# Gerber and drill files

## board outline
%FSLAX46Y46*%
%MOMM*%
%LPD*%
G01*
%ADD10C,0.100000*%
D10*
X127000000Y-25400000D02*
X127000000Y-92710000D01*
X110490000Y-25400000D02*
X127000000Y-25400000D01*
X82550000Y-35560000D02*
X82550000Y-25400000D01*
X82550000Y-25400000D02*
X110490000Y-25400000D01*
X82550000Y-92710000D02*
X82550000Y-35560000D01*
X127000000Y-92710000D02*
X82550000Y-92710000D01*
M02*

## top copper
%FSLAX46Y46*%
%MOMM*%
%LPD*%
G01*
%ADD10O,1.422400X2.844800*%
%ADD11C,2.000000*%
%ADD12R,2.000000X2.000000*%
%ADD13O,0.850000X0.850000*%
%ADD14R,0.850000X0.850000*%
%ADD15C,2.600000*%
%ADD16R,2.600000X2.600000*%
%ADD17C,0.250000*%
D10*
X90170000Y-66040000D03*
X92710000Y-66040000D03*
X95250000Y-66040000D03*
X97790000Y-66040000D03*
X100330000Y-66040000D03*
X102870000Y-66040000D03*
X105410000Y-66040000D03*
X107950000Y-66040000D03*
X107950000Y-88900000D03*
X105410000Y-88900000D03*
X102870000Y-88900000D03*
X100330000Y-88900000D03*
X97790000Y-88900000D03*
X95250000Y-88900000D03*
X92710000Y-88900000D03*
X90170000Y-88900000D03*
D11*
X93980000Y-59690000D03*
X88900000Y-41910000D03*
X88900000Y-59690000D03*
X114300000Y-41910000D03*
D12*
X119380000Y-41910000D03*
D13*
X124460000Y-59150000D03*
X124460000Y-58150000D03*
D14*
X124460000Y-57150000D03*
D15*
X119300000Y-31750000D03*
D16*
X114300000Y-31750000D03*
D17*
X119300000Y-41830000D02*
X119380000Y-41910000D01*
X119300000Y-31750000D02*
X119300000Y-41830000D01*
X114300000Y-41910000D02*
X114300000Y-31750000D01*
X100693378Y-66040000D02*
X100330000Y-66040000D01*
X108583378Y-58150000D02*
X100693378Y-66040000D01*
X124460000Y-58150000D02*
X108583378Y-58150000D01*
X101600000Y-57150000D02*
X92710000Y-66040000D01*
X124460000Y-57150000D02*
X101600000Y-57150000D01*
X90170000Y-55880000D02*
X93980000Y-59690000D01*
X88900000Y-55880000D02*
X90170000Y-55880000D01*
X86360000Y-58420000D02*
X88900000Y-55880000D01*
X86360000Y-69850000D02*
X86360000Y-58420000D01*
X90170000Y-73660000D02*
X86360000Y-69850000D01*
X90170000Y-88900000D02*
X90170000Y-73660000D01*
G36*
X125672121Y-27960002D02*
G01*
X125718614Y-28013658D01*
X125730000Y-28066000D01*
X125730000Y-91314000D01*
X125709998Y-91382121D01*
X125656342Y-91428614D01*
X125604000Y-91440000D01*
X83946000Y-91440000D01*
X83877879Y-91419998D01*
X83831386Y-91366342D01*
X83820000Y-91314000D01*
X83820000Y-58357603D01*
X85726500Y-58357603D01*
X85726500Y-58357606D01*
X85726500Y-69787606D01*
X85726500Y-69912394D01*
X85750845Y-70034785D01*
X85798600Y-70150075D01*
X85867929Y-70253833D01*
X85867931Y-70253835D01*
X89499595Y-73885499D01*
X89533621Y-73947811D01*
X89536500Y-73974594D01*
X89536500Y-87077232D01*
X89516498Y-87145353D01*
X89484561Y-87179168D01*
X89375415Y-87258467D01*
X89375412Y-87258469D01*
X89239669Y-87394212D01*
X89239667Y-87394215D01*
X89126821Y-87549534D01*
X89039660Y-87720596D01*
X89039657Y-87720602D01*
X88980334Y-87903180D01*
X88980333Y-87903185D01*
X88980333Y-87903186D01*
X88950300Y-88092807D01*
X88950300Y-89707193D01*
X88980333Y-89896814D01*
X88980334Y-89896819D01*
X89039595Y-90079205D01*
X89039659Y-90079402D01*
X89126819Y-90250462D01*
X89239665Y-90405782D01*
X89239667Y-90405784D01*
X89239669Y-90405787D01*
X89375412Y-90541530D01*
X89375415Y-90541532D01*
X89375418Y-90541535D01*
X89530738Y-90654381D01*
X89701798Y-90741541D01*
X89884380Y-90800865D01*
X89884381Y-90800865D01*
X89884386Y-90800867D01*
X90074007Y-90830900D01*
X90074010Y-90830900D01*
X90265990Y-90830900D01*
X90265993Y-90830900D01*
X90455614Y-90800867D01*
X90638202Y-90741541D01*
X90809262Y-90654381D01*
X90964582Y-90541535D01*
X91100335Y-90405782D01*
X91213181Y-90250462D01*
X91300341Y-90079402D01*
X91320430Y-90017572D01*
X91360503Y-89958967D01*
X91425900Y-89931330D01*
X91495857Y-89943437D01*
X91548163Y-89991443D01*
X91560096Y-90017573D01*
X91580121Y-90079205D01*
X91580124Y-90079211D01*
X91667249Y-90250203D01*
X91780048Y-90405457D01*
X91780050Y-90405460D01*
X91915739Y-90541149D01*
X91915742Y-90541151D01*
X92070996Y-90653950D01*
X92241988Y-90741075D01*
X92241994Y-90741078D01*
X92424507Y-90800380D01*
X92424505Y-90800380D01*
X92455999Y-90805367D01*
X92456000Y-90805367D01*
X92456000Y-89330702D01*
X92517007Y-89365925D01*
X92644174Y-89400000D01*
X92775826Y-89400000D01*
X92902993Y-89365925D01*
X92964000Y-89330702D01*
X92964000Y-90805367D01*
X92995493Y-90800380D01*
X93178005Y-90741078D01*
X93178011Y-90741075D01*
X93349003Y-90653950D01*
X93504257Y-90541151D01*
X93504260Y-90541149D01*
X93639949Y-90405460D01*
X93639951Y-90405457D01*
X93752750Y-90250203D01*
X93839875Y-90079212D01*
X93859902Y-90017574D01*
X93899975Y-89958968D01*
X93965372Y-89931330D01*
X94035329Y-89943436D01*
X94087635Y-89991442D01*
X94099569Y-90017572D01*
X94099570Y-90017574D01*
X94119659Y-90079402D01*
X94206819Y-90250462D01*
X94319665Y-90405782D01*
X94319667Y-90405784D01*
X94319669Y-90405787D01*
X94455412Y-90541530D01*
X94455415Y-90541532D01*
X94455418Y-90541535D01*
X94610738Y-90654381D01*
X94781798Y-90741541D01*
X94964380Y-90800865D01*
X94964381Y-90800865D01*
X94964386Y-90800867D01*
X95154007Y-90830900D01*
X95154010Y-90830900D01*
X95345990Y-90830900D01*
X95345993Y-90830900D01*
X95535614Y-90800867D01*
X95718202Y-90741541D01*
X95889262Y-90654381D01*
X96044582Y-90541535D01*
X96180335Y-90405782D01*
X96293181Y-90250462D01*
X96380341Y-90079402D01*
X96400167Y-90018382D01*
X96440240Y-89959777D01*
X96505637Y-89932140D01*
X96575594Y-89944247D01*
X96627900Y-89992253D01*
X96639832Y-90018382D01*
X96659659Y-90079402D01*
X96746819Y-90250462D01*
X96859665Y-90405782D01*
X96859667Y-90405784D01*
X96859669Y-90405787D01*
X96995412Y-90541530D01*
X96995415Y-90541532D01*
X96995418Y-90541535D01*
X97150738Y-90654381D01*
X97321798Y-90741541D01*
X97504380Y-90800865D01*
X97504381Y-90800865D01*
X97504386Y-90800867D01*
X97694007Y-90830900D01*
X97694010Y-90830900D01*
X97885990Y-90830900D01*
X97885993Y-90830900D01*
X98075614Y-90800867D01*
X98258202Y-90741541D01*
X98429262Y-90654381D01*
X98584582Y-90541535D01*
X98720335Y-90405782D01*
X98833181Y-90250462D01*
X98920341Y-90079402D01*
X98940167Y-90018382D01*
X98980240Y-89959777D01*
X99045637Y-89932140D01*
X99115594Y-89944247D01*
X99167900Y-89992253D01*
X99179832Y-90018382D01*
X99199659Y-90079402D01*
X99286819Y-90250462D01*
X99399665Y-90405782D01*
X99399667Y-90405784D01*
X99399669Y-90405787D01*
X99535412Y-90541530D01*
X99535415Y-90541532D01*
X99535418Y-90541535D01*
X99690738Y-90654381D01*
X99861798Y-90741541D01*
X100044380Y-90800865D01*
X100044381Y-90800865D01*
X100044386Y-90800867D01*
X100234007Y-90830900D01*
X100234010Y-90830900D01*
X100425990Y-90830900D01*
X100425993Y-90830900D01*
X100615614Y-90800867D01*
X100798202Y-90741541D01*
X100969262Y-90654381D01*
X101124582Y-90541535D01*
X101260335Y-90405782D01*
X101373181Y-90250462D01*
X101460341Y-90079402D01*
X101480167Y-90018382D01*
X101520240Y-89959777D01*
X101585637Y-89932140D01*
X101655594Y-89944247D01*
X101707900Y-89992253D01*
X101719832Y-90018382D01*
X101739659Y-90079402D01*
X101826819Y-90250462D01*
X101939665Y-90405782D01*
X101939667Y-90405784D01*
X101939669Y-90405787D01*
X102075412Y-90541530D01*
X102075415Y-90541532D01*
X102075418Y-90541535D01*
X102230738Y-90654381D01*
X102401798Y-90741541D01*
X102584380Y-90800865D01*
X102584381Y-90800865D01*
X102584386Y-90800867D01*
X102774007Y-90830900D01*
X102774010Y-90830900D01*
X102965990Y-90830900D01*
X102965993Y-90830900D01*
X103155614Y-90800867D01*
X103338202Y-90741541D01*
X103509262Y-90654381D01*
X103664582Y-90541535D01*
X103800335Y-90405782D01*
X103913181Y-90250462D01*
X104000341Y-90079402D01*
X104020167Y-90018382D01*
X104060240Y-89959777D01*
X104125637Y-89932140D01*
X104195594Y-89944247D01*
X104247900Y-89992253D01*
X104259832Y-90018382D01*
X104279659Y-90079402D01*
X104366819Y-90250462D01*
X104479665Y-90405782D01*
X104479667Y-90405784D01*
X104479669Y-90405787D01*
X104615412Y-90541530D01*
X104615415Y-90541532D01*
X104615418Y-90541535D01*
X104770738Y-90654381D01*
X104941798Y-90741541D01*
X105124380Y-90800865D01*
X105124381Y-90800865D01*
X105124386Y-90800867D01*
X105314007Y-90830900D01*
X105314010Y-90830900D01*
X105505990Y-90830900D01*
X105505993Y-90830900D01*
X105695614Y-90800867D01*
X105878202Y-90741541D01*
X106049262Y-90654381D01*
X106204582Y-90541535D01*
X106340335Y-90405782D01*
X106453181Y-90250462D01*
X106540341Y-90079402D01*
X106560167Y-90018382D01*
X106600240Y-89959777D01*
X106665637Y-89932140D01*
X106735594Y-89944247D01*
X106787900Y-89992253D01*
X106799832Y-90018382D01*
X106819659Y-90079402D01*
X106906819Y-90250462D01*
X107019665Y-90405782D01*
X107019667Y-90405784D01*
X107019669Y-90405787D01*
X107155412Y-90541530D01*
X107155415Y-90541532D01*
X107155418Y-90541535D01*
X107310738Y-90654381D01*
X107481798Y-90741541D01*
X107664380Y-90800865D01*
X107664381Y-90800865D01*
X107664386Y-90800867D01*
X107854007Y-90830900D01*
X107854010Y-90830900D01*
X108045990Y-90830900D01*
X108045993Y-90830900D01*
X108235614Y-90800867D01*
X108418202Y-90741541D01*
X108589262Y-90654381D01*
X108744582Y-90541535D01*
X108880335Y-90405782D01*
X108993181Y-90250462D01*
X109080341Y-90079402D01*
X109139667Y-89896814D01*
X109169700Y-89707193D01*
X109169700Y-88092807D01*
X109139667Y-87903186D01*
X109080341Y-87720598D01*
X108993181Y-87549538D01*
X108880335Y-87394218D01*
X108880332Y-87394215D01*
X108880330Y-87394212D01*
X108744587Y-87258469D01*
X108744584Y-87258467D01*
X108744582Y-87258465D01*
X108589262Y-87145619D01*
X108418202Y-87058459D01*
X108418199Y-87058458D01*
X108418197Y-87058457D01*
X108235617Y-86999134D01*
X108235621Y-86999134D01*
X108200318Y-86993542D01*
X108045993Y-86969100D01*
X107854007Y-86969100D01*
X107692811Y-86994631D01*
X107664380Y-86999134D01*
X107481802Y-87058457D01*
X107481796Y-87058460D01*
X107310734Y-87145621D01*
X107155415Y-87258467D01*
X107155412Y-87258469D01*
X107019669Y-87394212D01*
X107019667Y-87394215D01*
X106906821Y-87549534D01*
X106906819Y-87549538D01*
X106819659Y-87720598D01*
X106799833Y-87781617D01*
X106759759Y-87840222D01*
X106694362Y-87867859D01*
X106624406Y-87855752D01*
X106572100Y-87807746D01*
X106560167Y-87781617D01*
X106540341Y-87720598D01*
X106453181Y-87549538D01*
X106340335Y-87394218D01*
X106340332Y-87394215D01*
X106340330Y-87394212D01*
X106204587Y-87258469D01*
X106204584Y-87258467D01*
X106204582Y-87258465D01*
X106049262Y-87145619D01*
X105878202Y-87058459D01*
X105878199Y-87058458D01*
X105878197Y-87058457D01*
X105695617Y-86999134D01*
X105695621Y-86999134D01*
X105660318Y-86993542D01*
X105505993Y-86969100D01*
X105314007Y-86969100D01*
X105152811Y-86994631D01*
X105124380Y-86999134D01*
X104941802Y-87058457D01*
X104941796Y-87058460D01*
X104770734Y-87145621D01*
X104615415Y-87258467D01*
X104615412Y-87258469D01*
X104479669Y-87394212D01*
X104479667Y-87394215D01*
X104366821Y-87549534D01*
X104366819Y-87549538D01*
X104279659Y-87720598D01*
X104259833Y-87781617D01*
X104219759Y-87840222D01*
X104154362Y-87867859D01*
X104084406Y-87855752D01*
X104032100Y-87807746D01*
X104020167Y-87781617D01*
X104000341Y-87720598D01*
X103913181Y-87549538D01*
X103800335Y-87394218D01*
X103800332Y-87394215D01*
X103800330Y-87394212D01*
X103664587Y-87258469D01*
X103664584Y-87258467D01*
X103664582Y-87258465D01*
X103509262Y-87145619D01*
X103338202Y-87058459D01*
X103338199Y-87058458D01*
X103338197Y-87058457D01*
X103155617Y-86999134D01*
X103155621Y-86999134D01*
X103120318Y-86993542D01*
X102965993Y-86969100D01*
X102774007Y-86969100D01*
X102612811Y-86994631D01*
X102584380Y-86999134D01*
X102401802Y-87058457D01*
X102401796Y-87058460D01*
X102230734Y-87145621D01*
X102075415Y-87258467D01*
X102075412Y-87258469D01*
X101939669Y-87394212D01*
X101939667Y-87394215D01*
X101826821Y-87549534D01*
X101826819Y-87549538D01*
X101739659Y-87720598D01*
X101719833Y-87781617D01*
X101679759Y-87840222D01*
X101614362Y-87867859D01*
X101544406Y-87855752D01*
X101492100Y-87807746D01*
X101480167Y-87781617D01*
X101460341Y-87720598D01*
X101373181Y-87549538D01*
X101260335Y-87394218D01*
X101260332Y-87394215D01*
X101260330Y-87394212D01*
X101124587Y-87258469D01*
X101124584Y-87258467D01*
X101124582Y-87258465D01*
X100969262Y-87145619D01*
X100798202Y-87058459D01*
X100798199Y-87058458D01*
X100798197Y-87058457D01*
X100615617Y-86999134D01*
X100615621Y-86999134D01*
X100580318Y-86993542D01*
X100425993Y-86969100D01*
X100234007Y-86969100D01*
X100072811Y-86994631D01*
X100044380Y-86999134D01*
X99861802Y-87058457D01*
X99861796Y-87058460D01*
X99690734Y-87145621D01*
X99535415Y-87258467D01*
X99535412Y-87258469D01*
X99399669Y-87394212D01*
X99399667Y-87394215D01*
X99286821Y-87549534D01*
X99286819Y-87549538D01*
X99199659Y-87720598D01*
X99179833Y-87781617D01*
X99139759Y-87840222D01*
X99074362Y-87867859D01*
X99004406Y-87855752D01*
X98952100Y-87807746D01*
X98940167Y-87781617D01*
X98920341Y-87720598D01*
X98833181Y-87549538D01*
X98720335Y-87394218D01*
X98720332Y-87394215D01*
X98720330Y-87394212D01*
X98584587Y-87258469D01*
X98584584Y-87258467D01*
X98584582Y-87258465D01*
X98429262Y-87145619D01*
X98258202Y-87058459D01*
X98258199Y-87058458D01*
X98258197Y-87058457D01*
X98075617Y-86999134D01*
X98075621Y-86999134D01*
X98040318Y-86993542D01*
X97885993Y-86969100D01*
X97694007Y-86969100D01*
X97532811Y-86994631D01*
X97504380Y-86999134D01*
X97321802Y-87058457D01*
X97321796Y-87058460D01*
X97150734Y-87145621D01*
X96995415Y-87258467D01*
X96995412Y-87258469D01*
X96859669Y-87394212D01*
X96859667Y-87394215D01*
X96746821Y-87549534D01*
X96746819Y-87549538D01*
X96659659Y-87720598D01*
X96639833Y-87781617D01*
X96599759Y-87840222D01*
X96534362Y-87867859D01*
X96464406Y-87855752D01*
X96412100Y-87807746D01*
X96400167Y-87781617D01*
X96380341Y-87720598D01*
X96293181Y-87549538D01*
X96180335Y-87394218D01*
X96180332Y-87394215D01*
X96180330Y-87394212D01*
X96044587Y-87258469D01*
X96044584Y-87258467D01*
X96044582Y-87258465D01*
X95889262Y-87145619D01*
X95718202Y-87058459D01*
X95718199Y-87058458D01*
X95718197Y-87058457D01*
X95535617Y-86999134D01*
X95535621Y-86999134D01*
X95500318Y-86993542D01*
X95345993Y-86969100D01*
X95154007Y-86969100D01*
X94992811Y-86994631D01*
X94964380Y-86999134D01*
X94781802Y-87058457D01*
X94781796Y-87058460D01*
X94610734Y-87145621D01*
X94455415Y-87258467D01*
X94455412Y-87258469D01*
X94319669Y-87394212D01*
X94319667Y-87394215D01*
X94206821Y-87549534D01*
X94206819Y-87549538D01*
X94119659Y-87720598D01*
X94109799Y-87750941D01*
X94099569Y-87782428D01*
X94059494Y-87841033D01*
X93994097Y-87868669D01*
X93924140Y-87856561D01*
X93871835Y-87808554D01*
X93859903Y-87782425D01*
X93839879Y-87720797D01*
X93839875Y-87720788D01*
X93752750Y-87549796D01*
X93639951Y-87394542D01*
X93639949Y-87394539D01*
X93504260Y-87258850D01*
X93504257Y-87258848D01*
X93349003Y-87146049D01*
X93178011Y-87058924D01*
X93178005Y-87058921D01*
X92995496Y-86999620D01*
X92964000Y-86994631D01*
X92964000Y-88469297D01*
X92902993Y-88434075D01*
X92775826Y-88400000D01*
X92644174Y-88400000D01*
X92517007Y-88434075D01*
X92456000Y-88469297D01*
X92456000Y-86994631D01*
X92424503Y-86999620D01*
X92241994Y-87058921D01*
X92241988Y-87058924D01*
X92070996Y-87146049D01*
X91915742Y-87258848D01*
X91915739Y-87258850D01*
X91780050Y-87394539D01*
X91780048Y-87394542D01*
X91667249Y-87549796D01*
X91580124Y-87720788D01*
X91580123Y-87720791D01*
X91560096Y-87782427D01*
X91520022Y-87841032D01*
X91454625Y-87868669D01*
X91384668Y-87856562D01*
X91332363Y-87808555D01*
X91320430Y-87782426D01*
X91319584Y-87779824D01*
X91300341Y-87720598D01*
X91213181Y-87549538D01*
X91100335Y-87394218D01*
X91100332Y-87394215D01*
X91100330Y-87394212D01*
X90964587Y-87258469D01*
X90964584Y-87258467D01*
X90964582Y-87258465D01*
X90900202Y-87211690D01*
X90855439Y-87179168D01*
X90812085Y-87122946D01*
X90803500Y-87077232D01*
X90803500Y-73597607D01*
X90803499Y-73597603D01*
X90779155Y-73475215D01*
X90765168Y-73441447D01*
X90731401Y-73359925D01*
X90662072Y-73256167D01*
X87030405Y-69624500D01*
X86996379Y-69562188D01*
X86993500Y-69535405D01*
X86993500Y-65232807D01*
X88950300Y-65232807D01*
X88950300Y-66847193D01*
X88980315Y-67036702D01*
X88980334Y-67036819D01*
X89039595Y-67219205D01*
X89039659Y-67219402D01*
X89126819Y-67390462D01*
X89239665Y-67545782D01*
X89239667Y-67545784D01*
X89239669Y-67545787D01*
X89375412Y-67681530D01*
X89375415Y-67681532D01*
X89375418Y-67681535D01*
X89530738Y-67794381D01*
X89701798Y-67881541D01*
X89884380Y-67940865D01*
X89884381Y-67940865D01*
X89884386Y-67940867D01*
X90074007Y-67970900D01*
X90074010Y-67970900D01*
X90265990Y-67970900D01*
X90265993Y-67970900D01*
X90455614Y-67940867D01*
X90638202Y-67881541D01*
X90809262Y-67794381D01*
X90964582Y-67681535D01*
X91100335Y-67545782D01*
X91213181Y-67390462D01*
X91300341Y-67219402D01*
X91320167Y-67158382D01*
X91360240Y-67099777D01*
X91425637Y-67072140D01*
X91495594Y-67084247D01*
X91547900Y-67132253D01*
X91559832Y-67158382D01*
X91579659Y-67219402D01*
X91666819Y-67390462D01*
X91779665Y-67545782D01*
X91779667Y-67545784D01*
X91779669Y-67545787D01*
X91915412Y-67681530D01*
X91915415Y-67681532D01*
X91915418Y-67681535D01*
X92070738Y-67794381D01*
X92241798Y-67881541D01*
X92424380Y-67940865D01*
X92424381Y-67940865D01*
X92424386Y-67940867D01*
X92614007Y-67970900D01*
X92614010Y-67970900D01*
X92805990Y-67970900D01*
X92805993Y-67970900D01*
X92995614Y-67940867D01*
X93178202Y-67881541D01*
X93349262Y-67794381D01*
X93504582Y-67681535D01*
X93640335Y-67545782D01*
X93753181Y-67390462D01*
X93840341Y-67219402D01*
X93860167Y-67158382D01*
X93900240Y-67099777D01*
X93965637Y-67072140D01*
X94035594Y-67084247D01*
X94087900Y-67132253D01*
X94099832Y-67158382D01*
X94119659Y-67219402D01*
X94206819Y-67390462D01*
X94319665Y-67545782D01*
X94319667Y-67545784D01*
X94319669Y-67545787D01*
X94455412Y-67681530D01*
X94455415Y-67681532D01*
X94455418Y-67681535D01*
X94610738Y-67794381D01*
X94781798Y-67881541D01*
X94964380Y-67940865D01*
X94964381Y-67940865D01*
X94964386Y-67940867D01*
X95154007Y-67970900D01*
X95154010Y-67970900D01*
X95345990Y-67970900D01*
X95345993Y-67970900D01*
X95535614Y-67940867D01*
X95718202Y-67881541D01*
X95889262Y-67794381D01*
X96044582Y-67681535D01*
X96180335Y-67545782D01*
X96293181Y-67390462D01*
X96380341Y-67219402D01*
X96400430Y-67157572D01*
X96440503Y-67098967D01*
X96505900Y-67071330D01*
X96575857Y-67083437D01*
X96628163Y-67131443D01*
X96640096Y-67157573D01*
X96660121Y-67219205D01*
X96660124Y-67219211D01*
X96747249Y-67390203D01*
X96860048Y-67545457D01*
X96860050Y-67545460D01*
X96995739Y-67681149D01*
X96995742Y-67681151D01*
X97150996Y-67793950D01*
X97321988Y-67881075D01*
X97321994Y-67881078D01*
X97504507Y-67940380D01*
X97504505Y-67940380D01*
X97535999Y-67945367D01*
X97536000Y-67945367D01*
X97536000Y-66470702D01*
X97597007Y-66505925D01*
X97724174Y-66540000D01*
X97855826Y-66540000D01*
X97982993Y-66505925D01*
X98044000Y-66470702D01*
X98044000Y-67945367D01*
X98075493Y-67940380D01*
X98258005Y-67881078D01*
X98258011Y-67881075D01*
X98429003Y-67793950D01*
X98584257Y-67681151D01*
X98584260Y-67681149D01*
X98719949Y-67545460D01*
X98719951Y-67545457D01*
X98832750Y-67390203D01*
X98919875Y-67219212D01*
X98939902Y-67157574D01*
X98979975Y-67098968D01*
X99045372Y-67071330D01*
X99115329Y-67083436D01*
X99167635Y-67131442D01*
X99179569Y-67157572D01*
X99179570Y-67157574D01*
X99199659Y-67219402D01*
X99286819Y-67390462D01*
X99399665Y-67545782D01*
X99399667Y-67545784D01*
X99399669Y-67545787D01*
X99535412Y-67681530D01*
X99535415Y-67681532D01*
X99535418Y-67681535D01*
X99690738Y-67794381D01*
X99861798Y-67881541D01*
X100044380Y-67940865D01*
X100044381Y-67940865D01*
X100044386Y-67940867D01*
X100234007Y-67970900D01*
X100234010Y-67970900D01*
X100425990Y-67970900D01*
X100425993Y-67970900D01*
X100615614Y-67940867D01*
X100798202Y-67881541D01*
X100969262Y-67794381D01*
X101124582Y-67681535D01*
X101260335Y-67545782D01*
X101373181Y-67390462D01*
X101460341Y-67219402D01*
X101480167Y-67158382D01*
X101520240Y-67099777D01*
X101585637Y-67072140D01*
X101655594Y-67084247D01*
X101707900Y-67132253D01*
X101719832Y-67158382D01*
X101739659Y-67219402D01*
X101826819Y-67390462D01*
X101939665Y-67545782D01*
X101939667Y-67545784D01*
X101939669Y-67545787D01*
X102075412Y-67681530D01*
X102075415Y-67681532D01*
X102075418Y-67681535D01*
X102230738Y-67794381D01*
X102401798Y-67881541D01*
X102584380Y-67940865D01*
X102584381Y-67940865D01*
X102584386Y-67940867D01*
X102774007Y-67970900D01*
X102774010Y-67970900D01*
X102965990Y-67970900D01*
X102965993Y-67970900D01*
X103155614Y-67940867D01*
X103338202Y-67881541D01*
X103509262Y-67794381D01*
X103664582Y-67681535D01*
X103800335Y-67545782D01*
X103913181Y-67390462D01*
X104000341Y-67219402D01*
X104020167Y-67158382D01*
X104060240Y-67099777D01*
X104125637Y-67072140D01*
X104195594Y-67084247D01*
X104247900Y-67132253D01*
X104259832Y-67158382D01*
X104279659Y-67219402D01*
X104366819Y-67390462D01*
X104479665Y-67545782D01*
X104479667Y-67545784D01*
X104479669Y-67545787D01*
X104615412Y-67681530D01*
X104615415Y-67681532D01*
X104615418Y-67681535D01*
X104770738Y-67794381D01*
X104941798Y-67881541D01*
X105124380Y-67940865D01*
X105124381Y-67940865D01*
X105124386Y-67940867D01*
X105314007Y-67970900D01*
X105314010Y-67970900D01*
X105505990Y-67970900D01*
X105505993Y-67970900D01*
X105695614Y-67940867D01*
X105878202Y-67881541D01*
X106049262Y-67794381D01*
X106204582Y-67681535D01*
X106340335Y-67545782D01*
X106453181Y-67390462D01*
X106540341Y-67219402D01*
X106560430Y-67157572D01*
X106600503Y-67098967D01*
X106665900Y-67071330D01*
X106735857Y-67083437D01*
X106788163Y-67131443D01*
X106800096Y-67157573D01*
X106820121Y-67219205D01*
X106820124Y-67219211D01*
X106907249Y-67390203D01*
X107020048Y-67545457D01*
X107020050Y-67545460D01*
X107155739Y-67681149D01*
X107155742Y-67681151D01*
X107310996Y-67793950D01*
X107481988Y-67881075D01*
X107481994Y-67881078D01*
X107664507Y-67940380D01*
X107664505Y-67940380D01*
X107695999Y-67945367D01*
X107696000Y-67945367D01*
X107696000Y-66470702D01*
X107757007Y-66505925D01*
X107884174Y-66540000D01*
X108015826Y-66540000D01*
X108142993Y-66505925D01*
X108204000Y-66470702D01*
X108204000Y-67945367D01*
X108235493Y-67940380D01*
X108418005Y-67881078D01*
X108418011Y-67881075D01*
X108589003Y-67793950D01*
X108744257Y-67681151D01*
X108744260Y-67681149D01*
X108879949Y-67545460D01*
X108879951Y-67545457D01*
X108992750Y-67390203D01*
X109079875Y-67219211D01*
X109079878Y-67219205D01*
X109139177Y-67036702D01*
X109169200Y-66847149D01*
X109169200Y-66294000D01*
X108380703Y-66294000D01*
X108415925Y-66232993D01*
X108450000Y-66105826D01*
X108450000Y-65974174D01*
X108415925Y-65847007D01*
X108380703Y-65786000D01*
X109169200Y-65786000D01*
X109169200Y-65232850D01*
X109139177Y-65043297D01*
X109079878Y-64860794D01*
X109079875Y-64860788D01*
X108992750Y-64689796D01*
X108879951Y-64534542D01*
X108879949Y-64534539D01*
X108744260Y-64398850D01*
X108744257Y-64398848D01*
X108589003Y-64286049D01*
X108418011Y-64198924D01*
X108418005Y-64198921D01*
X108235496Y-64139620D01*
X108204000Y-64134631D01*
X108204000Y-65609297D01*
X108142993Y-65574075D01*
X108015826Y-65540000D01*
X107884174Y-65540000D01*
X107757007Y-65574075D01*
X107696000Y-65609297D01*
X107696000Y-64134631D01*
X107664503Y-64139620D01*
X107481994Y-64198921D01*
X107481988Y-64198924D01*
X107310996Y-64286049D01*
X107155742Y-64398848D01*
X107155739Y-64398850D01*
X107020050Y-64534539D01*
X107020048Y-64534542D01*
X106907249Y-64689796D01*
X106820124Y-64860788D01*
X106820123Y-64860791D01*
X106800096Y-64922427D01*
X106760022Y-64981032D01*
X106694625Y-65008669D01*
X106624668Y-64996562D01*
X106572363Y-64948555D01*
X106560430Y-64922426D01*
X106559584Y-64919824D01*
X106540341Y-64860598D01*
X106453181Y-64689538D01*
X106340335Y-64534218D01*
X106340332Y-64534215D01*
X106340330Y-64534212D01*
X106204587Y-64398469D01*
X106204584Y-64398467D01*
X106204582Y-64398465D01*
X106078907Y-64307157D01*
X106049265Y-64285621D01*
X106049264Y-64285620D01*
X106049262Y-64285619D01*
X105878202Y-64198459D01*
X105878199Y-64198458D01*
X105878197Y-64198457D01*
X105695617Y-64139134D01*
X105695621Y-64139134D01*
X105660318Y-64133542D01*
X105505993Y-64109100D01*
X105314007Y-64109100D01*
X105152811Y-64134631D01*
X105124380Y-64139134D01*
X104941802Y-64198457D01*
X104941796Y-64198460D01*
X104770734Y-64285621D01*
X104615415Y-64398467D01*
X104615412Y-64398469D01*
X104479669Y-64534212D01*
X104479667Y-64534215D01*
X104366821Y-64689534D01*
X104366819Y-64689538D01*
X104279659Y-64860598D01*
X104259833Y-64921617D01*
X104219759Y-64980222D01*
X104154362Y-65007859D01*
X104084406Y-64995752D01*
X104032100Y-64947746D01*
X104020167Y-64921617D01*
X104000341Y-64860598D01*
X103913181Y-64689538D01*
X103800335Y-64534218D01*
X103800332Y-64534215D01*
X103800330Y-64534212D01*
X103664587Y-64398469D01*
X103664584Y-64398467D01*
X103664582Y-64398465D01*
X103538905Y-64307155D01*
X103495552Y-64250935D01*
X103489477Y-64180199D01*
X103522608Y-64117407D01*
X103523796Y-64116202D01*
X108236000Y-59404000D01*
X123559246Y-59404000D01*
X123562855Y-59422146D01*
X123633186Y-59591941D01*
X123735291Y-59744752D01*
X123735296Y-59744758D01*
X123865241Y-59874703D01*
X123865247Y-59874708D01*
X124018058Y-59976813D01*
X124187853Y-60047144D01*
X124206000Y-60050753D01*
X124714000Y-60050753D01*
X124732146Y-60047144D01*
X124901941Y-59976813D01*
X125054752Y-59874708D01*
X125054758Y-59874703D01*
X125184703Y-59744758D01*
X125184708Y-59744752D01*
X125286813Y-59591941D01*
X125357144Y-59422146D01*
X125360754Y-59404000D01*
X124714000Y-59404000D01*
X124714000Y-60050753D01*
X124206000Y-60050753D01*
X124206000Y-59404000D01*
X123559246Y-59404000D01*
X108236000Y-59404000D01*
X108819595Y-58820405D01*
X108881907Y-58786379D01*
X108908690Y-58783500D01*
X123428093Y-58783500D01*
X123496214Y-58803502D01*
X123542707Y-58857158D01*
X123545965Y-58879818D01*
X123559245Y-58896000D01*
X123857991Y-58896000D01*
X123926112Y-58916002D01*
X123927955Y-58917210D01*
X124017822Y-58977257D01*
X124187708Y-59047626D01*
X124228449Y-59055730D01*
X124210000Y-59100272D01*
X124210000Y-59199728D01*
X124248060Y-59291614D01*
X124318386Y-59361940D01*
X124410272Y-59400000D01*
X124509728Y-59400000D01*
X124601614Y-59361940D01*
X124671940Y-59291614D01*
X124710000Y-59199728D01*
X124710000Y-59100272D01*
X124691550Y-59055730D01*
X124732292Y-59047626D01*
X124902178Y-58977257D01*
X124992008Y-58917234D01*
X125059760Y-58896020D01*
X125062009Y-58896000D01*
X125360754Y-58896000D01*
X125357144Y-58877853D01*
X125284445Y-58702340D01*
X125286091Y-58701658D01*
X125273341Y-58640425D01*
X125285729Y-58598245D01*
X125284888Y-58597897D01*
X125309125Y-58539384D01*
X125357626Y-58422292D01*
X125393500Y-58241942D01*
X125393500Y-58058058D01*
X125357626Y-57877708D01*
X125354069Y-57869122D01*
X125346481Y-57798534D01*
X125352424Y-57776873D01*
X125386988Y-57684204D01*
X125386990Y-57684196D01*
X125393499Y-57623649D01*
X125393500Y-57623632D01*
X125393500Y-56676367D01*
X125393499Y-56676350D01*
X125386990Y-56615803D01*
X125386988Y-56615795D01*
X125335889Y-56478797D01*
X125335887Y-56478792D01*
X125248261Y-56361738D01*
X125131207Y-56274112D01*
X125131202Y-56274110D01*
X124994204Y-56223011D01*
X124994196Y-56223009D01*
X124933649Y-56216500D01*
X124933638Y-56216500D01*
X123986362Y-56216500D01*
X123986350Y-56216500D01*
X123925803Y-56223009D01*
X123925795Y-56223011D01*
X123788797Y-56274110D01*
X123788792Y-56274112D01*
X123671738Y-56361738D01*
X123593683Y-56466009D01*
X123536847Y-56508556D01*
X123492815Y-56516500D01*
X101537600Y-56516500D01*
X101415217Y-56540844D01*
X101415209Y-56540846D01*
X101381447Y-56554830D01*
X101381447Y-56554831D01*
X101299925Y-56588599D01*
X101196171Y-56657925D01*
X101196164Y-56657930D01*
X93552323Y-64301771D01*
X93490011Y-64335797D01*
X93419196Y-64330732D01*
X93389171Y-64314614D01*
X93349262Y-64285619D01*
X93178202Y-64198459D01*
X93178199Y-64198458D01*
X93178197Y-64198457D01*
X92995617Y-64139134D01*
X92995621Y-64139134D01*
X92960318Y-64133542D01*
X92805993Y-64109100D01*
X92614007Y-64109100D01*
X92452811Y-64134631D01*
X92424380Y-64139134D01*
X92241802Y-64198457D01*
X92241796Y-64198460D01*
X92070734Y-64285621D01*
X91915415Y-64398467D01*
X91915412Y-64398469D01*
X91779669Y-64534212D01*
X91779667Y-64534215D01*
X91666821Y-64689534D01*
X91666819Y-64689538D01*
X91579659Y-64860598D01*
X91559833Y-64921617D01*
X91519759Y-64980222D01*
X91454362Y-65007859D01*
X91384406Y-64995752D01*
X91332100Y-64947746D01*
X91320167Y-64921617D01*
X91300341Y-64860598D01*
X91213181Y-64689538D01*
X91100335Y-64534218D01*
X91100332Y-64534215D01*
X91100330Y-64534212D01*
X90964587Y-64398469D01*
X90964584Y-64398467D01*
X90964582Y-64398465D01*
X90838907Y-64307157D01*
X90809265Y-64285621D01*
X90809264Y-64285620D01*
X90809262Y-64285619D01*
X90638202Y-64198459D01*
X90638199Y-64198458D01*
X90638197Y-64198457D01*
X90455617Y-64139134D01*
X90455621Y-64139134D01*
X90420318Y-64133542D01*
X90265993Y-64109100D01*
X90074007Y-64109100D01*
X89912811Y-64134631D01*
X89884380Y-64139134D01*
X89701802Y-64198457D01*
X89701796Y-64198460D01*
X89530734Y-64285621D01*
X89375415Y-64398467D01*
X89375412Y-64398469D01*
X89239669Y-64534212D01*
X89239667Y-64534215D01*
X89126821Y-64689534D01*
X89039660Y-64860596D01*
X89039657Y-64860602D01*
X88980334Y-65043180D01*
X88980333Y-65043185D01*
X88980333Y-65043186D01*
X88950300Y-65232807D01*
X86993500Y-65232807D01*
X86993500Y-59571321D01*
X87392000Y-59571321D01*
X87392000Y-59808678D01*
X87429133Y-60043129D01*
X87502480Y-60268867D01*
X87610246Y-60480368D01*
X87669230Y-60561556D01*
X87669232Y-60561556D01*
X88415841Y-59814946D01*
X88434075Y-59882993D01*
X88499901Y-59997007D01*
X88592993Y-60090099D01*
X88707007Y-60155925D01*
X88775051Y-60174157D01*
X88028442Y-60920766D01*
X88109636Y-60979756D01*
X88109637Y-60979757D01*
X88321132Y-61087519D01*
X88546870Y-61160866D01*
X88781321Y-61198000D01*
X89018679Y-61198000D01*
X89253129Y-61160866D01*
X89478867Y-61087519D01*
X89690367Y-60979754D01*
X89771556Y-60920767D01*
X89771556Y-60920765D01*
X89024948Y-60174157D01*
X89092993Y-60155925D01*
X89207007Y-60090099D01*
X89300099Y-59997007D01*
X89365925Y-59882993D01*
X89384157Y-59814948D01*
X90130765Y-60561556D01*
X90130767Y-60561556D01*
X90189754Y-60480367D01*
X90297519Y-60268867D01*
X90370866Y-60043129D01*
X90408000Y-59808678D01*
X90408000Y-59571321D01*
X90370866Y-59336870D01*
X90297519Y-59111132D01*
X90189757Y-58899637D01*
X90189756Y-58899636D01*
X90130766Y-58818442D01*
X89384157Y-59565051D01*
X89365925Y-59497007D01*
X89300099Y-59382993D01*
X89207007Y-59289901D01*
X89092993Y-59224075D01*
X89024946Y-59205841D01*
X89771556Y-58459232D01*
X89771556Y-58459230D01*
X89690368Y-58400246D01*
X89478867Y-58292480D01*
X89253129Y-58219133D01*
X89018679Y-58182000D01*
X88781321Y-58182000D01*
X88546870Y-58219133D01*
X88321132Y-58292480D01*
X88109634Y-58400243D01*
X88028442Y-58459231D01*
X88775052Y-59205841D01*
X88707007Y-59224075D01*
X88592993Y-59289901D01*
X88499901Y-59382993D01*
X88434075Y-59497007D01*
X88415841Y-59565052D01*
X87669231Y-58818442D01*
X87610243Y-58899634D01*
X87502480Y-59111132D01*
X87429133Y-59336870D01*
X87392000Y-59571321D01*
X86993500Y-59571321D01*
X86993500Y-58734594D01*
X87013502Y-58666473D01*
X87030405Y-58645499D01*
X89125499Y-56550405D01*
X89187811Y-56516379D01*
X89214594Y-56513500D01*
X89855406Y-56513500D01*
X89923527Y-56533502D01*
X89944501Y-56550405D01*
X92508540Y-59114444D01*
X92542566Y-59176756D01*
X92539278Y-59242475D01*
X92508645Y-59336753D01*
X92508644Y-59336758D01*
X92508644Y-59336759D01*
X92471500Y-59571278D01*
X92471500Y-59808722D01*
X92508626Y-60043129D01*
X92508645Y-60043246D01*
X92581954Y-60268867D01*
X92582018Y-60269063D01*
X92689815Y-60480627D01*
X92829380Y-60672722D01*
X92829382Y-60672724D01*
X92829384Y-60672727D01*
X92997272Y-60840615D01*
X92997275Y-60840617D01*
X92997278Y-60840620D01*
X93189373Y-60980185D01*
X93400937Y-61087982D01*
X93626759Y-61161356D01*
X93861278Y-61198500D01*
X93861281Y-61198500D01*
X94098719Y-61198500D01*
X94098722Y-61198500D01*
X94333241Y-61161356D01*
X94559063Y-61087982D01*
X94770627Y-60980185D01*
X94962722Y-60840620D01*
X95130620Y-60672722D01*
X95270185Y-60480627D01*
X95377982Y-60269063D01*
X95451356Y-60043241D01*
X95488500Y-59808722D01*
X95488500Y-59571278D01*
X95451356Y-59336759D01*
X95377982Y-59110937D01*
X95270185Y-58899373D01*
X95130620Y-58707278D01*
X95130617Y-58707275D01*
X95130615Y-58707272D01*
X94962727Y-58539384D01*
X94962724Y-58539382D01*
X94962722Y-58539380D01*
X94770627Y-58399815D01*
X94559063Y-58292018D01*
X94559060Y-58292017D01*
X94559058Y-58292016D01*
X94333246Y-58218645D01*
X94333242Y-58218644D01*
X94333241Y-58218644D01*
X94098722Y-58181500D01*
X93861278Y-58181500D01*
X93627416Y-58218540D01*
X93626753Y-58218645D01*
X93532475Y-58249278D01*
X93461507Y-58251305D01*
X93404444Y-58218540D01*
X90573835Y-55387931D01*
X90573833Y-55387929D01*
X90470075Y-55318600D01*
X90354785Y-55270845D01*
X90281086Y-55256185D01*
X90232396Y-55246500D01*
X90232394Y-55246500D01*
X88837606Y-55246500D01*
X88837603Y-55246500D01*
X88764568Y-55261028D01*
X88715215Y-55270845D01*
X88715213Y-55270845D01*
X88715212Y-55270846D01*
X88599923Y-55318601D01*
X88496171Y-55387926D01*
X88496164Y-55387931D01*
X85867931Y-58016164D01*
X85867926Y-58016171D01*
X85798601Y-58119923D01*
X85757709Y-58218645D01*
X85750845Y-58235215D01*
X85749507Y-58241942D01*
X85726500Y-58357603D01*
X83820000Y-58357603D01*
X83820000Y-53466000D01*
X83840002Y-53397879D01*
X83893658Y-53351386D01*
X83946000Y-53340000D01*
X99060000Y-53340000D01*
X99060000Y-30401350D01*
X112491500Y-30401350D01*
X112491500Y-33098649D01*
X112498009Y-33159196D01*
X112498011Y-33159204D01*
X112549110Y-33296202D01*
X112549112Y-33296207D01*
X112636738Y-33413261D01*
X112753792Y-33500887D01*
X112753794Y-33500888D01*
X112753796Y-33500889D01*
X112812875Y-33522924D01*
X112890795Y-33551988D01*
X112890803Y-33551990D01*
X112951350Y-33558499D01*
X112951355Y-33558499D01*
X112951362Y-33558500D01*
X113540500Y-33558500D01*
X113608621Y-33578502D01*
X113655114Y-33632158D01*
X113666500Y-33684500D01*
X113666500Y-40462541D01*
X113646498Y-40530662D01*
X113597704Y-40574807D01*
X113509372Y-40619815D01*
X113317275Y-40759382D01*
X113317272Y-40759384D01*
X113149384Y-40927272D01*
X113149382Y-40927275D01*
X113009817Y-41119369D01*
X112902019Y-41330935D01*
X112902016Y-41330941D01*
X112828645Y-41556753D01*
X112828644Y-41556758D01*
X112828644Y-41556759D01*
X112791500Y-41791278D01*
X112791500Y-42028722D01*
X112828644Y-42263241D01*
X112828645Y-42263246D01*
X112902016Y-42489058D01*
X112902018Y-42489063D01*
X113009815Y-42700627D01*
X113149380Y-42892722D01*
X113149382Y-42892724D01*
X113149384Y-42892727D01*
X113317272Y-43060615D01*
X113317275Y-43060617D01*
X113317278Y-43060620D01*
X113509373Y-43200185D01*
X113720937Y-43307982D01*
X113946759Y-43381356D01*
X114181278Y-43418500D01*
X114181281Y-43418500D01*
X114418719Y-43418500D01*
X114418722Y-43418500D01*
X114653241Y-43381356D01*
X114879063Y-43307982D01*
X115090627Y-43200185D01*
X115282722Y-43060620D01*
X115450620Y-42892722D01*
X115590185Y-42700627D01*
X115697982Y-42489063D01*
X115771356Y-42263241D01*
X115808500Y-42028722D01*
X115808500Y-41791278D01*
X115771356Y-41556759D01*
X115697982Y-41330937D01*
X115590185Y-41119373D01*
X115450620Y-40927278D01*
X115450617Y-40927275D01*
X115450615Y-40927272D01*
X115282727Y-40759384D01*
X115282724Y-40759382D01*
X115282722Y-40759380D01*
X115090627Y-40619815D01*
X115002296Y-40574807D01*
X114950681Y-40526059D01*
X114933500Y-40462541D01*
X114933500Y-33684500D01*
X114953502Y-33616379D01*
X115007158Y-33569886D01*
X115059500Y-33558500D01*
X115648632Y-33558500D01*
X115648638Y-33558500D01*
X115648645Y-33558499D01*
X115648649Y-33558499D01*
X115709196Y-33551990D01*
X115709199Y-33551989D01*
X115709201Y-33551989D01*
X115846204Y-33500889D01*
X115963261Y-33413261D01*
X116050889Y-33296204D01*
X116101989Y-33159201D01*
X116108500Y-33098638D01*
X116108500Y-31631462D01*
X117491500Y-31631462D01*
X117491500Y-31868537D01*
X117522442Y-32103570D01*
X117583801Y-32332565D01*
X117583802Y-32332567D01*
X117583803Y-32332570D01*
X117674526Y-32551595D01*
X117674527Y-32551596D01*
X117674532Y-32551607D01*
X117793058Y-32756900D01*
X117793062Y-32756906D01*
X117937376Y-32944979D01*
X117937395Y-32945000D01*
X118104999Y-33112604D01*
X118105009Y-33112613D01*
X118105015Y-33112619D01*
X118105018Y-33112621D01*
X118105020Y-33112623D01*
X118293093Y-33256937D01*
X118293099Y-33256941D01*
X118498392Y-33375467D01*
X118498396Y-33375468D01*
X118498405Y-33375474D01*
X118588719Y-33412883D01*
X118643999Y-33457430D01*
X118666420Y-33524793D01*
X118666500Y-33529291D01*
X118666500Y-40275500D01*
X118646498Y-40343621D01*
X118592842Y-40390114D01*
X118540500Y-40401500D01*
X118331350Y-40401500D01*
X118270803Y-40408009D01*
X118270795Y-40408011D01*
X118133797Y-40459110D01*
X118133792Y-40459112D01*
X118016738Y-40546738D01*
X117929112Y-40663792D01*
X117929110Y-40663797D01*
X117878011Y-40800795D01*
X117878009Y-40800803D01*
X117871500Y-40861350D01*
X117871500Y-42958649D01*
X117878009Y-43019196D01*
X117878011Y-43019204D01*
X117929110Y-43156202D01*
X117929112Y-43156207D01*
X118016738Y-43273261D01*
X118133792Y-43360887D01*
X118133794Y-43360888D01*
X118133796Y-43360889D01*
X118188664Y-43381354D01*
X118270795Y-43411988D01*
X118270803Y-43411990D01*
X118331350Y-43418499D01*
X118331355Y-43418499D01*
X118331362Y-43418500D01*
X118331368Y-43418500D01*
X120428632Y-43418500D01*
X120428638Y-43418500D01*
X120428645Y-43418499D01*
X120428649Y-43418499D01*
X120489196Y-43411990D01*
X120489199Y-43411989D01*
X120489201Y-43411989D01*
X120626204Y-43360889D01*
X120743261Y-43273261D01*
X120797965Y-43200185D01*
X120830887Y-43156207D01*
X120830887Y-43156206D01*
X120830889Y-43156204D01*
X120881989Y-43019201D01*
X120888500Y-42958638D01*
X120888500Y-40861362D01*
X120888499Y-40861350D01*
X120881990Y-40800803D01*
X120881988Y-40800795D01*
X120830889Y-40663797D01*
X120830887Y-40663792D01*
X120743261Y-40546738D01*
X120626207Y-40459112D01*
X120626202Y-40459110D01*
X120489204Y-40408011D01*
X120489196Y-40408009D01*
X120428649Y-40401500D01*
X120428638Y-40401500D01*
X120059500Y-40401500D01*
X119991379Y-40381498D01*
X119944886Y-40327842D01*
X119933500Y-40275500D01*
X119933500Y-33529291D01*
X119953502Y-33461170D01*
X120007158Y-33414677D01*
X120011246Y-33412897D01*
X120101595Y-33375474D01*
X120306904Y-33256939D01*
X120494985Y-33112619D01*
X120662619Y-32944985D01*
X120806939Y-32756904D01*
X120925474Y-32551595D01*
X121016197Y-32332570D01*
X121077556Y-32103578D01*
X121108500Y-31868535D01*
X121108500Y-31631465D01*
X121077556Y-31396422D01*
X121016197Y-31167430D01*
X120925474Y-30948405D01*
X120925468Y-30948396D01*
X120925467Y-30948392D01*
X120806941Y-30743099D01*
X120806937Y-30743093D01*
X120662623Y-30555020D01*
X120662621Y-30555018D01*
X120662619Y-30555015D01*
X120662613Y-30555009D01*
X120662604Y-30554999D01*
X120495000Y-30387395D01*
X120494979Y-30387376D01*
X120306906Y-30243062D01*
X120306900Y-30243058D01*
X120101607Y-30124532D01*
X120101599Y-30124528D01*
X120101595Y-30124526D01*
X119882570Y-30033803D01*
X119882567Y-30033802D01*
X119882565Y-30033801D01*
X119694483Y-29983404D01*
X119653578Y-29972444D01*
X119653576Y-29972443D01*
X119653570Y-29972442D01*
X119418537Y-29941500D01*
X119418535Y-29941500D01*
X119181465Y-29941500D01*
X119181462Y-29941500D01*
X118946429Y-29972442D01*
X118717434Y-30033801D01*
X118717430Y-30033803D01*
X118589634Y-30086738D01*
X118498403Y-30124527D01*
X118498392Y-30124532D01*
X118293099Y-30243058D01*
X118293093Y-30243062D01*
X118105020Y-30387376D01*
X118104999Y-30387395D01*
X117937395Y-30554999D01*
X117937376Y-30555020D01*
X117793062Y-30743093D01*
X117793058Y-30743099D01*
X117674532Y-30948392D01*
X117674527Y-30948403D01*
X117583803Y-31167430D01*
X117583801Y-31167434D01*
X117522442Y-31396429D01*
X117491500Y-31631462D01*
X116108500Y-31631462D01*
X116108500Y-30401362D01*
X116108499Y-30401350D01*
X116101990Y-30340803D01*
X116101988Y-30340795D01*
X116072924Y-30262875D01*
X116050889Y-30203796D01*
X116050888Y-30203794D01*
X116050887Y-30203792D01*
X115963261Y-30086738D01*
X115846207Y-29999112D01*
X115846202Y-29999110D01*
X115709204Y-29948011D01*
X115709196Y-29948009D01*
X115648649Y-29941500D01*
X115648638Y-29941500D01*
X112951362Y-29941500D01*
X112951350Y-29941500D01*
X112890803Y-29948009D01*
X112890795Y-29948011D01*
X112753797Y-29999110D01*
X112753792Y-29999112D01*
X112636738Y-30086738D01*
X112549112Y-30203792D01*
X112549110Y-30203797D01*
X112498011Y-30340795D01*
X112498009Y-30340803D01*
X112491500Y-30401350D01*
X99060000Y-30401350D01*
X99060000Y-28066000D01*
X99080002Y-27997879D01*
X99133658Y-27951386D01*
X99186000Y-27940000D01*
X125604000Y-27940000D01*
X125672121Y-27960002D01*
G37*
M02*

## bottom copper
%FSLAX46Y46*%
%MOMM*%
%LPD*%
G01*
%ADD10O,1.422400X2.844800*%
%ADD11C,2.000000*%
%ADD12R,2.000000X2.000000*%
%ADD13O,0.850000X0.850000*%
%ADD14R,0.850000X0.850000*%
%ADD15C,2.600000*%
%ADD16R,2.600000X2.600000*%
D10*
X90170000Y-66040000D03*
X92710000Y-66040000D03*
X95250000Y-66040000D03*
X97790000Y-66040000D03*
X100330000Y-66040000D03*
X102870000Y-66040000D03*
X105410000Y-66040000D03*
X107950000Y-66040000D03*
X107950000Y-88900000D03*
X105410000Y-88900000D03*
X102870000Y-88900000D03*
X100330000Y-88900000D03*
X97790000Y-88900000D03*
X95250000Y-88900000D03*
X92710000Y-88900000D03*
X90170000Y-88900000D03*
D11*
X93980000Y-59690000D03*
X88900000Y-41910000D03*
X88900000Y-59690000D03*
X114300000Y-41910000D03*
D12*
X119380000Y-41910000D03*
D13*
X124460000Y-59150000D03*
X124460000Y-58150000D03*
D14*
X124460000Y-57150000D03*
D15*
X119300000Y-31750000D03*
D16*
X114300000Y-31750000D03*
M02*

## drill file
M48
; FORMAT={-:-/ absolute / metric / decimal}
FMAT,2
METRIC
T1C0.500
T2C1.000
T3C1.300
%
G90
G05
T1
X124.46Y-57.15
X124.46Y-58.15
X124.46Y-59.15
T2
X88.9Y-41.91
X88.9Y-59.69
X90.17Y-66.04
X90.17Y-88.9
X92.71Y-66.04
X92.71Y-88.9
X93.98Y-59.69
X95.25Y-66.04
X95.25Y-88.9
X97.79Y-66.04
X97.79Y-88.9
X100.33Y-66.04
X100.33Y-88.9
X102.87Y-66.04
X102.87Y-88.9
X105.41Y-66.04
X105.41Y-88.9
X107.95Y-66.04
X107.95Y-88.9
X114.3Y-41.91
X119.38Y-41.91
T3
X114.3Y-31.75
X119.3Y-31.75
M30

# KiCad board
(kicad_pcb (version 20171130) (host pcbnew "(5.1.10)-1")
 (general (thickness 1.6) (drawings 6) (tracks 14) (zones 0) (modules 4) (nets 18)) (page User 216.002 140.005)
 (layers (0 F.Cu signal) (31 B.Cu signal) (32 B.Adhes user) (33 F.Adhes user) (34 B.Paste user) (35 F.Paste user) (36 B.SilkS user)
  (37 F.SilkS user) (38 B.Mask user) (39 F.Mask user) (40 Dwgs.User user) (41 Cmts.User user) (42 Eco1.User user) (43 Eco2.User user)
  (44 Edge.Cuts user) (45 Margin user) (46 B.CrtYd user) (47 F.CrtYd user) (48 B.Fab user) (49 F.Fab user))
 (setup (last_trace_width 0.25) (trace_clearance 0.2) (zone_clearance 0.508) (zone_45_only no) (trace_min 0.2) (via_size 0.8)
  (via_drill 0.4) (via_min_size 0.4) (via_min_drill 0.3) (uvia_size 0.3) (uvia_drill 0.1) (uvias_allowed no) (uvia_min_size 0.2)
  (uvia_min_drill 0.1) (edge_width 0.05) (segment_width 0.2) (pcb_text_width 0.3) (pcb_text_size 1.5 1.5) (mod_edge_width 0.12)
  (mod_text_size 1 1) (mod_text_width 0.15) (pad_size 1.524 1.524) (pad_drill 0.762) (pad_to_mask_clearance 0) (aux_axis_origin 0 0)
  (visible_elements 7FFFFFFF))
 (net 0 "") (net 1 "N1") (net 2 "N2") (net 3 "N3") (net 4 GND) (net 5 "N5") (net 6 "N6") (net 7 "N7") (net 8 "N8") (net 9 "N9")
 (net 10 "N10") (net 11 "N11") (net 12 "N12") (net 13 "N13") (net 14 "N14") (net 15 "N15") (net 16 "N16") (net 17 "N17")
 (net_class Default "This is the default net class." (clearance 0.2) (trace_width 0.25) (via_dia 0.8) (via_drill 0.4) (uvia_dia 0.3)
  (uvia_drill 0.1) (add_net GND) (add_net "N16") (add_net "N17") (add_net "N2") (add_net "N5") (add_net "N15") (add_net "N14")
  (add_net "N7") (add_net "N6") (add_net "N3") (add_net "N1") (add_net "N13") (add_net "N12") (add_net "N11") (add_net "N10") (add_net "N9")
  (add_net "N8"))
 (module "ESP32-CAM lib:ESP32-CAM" (layer F.Cu) (at 100.33 77.47 90)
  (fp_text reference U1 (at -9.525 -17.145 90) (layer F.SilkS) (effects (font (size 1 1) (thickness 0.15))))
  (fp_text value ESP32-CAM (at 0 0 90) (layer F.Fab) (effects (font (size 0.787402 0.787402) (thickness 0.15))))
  (pad P$16 thru_hole oval (at 11.43 -10.16 90) (size 2.8448 1.4224) (drill 1) (layers *.Cu *.Mask) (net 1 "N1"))
  (pad P$15 thru_hole oval (at 11.43 -7.62 90) (size 2.8448 1.4224) (drill 1) (layers *.Cu *.Mask) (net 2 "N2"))
  (pad P$14 thru_hole oval (at 11.43 -5.08 90) (size 2.8448 1.4224) (drill 1) (layers *.Cu *.Mask) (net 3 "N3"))
  (pad P$13 thru_hole oval (at 11.43 -2.54 90) (size 2.8448 1.4224) (drill 1) (layers *.Cu *.Mask) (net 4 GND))
  (pad P$12 thru_hole oval (at 11.43 0 90) (size 2.8448 1.4224) (drill 1) (layers *.Cu *.Mask) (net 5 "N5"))
  (pad P$11 thru_hole oval (at 11.43 2.54 90) (size 2.8448 1.4224) (drill 1) (layers *.Cu *.Mask) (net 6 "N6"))
  (pad P$10 thru_hole oval (at 11.43 5.08 90) (size 2.8448 1.4224) (drill 1) (layers *.Cu *.Mask) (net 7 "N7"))
  (pad P$9 thru_hole oval (at 11.43 7.62 90) (size 2.8448 1.4224) (drill 1) (layers *.Cu *.Mask) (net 4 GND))
  (pad P$8 thru_hole oval (at -11.43 7.62 90) (size 2.8448 1.4224) (drill 1) (layers *.Cu *.Mask) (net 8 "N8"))
  (pad P$7 thru_hole oval (at -11.43 5.08 90) (size 2.8448 1.4224) (drill 1) (layers *.Cu *.Mask) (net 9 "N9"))
  (pad P$6 thru_hole oval (at -11.43 2.54 90) (size 2.8448 1.4224) (drill 1) (layers *.Cu *.Mask) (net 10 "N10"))
  (pad P$5 thru_hole oval (at -11.43 0 90) (size 2.8448 1.4224) (drill 1) (layers *.Cu *.Mask) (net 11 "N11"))
  (pad P$4 thru_hole oval (at -11.43 -2.54 90) (size 2.8448 1.4224) (drill 1) (layers *.Cu *.Mask) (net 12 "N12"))
  (pad P$3 thru_hole oval (at -11.43 -5.08 90) (size 2.8448 1.4224) (drill 1) (layers *.Cu *.Mask) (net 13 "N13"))
  (pad P$2 thru_hole oval (at -11.43 -7.62 90) (size 2.8448 1.4224) (drill 1) (layers *.Cu *.Mask) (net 4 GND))
  (pad P$1 thru_hole oval (at -11.43 -10.16 90) (size 2.8448 1.4224) (drill 1) (layers *.Cu *.Mask) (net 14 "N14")))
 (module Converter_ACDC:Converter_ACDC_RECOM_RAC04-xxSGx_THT (layer F.Cu) (at 119.38 41.91 270)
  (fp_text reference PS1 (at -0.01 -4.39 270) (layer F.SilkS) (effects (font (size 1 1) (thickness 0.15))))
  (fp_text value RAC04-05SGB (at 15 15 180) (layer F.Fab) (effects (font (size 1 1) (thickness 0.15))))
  (pad 5 thru_hole circle (at 17.78 25.4) (size 2 2) (drill 1) (layers *.Cu *.Mask) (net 14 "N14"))
  (pad 3 thru_hole circle (at 0 30.48 90) (size 2 2) (drill 1) (layers *.Cu *.Mask) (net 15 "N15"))
  (pad 4 thru_hole circle (at 17.78 30.48) (size 2 2) (drill 1) (layers *.Cu *.Mask) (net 4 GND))
  (pad 2 thru_hole circle (at 0 5.08) (size 2 2) (drill 1) (layers *.Cu *.Mask) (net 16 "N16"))
  (pad 1 thru_hole rect (at 0 0) (size 2 2) (drill 1) (layers *.Cu *.Mask) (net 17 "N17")))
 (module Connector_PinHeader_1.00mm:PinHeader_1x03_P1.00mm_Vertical (layer F.Cu) (at 124.46 57.15)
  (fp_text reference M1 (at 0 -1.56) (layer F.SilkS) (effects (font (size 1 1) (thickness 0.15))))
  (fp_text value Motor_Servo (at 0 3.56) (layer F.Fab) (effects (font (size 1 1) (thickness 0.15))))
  (pad 3 thru_hole oval (at 0 2) (size 0.85 0.85) (drill 0.5) (layers *.Cu *.Mask) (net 4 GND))
  (pad 2 thru_hole oval (at 0 1) (size 0.85 0.85) (drill 0.5) (layers *.Cu *.Mask) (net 5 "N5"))
  (pad 1 thru_hole rect (at 0 0) (size 0.85 0.85) (drill 0.5) (layers *.Cu *.Mask) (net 2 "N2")))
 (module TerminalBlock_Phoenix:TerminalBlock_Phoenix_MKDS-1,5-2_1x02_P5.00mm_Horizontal (layer F.Cu) (at 114.3 31.75)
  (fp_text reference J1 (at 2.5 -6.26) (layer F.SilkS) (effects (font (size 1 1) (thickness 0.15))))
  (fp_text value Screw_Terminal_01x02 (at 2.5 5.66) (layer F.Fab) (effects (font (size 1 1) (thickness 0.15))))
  (pad 2 thru_hole circle (at 5 0) (size 2.6 2.6) (drill 1.3) (layers *.Cu *.Mask) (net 17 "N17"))
  (pad 1 thru_hole rect (at 0 0) (size 2.6 2.6) (drill 1.3) (layers *.Cu *.Mask) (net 16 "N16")))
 (gr_line (start 127 25.4) (end 127 92.71) (layer Edge.Cuts) (width 0.1))
 (gr_line (start 110.49 25.4) (end 127 25.4) (layer Edge.Cuts) (width 0.1))
 (gr_line (start 82.55 35.56) (end 82.55 25.4) (layer Edge.Cuts) (width 0.1))
 (gr_line (start 82.55 25.4) (end 110.49 25.4) (layer Edge.Cuts) (width 0.1))
 (gr_line (start 82.55 92.71) (end 82.55 35.56) (layer Edge.Cuts) (width 0.1))
 (gr_line (start 127 92.71) (end 82.55 92.71) (layer Edge.Cuts) (width 0.1))
 (segment (start 119.3 41.83) (end 119.38 41.91) (width 0.25) (layer F.Cu) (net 17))
 (segment (start 119.3 31.75) (end 119.3 41.83) (width 0.25) (layer F.Cu) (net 17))
 (segment (start 114.3 41.91) (end 114.3 31.75) (width 0.25) (layer F.Cu) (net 16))
 (segment (start 100.693378 66.04) (end 100.33 66.04) (width 0.25) (layer F.Cu) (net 5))
 (segment (start 108.583378 58.15) (end 100.693378 66.04) (width 0.25) (layer F.Cu) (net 5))
 (segment (start 124.46 58.15) (end 108.583378 58.15) (width 0.25) (layer F.Cu) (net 5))
 (segment (start 101.6 57.15) (end 92.71 66.04) (width 0.25) (layer F.Cu) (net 2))
 (segment (start 124.46 57.15) (end 101.6 57.15) (width 0.25) (layer F.Cu) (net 2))
 (segment (start 90.17 55.88) (end 93.98 59.69) (width 0.25) (layer F.Cu) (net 14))
 (segment (start 88.9 55.88) (end 90.17 55.88) (width 0.25) (layer F.Cu) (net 14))
 (segment (start 86.36 58.42) (end 88.9 55.88) (width 0.25) (layer F.Cu) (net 14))
 (segment (start 86.36 69.85) (end 86.36 58.42) (width 0.25) (layer F.Cu) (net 14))
 (segment (start 90.17 73.66) (end 86.36 69.85) (width 0.25) (layer F.Cu) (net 14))
 (segment (start 90.17 88.9) (end 90.17 73.66) (width 0.25) (layer F.Cu) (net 14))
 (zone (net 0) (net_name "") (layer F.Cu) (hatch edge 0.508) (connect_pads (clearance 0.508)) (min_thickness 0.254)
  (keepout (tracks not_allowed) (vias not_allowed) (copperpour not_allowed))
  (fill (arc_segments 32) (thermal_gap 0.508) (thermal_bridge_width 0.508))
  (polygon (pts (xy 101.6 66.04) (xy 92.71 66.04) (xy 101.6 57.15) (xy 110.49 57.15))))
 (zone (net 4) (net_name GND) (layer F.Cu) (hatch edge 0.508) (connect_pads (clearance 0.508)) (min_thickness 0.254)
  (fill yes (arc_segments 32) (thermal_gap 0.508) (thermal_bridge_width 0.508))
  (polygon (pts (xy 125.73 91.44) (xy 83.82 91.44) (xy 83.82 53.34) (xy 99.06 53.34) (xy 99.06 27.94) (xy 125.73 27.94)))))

